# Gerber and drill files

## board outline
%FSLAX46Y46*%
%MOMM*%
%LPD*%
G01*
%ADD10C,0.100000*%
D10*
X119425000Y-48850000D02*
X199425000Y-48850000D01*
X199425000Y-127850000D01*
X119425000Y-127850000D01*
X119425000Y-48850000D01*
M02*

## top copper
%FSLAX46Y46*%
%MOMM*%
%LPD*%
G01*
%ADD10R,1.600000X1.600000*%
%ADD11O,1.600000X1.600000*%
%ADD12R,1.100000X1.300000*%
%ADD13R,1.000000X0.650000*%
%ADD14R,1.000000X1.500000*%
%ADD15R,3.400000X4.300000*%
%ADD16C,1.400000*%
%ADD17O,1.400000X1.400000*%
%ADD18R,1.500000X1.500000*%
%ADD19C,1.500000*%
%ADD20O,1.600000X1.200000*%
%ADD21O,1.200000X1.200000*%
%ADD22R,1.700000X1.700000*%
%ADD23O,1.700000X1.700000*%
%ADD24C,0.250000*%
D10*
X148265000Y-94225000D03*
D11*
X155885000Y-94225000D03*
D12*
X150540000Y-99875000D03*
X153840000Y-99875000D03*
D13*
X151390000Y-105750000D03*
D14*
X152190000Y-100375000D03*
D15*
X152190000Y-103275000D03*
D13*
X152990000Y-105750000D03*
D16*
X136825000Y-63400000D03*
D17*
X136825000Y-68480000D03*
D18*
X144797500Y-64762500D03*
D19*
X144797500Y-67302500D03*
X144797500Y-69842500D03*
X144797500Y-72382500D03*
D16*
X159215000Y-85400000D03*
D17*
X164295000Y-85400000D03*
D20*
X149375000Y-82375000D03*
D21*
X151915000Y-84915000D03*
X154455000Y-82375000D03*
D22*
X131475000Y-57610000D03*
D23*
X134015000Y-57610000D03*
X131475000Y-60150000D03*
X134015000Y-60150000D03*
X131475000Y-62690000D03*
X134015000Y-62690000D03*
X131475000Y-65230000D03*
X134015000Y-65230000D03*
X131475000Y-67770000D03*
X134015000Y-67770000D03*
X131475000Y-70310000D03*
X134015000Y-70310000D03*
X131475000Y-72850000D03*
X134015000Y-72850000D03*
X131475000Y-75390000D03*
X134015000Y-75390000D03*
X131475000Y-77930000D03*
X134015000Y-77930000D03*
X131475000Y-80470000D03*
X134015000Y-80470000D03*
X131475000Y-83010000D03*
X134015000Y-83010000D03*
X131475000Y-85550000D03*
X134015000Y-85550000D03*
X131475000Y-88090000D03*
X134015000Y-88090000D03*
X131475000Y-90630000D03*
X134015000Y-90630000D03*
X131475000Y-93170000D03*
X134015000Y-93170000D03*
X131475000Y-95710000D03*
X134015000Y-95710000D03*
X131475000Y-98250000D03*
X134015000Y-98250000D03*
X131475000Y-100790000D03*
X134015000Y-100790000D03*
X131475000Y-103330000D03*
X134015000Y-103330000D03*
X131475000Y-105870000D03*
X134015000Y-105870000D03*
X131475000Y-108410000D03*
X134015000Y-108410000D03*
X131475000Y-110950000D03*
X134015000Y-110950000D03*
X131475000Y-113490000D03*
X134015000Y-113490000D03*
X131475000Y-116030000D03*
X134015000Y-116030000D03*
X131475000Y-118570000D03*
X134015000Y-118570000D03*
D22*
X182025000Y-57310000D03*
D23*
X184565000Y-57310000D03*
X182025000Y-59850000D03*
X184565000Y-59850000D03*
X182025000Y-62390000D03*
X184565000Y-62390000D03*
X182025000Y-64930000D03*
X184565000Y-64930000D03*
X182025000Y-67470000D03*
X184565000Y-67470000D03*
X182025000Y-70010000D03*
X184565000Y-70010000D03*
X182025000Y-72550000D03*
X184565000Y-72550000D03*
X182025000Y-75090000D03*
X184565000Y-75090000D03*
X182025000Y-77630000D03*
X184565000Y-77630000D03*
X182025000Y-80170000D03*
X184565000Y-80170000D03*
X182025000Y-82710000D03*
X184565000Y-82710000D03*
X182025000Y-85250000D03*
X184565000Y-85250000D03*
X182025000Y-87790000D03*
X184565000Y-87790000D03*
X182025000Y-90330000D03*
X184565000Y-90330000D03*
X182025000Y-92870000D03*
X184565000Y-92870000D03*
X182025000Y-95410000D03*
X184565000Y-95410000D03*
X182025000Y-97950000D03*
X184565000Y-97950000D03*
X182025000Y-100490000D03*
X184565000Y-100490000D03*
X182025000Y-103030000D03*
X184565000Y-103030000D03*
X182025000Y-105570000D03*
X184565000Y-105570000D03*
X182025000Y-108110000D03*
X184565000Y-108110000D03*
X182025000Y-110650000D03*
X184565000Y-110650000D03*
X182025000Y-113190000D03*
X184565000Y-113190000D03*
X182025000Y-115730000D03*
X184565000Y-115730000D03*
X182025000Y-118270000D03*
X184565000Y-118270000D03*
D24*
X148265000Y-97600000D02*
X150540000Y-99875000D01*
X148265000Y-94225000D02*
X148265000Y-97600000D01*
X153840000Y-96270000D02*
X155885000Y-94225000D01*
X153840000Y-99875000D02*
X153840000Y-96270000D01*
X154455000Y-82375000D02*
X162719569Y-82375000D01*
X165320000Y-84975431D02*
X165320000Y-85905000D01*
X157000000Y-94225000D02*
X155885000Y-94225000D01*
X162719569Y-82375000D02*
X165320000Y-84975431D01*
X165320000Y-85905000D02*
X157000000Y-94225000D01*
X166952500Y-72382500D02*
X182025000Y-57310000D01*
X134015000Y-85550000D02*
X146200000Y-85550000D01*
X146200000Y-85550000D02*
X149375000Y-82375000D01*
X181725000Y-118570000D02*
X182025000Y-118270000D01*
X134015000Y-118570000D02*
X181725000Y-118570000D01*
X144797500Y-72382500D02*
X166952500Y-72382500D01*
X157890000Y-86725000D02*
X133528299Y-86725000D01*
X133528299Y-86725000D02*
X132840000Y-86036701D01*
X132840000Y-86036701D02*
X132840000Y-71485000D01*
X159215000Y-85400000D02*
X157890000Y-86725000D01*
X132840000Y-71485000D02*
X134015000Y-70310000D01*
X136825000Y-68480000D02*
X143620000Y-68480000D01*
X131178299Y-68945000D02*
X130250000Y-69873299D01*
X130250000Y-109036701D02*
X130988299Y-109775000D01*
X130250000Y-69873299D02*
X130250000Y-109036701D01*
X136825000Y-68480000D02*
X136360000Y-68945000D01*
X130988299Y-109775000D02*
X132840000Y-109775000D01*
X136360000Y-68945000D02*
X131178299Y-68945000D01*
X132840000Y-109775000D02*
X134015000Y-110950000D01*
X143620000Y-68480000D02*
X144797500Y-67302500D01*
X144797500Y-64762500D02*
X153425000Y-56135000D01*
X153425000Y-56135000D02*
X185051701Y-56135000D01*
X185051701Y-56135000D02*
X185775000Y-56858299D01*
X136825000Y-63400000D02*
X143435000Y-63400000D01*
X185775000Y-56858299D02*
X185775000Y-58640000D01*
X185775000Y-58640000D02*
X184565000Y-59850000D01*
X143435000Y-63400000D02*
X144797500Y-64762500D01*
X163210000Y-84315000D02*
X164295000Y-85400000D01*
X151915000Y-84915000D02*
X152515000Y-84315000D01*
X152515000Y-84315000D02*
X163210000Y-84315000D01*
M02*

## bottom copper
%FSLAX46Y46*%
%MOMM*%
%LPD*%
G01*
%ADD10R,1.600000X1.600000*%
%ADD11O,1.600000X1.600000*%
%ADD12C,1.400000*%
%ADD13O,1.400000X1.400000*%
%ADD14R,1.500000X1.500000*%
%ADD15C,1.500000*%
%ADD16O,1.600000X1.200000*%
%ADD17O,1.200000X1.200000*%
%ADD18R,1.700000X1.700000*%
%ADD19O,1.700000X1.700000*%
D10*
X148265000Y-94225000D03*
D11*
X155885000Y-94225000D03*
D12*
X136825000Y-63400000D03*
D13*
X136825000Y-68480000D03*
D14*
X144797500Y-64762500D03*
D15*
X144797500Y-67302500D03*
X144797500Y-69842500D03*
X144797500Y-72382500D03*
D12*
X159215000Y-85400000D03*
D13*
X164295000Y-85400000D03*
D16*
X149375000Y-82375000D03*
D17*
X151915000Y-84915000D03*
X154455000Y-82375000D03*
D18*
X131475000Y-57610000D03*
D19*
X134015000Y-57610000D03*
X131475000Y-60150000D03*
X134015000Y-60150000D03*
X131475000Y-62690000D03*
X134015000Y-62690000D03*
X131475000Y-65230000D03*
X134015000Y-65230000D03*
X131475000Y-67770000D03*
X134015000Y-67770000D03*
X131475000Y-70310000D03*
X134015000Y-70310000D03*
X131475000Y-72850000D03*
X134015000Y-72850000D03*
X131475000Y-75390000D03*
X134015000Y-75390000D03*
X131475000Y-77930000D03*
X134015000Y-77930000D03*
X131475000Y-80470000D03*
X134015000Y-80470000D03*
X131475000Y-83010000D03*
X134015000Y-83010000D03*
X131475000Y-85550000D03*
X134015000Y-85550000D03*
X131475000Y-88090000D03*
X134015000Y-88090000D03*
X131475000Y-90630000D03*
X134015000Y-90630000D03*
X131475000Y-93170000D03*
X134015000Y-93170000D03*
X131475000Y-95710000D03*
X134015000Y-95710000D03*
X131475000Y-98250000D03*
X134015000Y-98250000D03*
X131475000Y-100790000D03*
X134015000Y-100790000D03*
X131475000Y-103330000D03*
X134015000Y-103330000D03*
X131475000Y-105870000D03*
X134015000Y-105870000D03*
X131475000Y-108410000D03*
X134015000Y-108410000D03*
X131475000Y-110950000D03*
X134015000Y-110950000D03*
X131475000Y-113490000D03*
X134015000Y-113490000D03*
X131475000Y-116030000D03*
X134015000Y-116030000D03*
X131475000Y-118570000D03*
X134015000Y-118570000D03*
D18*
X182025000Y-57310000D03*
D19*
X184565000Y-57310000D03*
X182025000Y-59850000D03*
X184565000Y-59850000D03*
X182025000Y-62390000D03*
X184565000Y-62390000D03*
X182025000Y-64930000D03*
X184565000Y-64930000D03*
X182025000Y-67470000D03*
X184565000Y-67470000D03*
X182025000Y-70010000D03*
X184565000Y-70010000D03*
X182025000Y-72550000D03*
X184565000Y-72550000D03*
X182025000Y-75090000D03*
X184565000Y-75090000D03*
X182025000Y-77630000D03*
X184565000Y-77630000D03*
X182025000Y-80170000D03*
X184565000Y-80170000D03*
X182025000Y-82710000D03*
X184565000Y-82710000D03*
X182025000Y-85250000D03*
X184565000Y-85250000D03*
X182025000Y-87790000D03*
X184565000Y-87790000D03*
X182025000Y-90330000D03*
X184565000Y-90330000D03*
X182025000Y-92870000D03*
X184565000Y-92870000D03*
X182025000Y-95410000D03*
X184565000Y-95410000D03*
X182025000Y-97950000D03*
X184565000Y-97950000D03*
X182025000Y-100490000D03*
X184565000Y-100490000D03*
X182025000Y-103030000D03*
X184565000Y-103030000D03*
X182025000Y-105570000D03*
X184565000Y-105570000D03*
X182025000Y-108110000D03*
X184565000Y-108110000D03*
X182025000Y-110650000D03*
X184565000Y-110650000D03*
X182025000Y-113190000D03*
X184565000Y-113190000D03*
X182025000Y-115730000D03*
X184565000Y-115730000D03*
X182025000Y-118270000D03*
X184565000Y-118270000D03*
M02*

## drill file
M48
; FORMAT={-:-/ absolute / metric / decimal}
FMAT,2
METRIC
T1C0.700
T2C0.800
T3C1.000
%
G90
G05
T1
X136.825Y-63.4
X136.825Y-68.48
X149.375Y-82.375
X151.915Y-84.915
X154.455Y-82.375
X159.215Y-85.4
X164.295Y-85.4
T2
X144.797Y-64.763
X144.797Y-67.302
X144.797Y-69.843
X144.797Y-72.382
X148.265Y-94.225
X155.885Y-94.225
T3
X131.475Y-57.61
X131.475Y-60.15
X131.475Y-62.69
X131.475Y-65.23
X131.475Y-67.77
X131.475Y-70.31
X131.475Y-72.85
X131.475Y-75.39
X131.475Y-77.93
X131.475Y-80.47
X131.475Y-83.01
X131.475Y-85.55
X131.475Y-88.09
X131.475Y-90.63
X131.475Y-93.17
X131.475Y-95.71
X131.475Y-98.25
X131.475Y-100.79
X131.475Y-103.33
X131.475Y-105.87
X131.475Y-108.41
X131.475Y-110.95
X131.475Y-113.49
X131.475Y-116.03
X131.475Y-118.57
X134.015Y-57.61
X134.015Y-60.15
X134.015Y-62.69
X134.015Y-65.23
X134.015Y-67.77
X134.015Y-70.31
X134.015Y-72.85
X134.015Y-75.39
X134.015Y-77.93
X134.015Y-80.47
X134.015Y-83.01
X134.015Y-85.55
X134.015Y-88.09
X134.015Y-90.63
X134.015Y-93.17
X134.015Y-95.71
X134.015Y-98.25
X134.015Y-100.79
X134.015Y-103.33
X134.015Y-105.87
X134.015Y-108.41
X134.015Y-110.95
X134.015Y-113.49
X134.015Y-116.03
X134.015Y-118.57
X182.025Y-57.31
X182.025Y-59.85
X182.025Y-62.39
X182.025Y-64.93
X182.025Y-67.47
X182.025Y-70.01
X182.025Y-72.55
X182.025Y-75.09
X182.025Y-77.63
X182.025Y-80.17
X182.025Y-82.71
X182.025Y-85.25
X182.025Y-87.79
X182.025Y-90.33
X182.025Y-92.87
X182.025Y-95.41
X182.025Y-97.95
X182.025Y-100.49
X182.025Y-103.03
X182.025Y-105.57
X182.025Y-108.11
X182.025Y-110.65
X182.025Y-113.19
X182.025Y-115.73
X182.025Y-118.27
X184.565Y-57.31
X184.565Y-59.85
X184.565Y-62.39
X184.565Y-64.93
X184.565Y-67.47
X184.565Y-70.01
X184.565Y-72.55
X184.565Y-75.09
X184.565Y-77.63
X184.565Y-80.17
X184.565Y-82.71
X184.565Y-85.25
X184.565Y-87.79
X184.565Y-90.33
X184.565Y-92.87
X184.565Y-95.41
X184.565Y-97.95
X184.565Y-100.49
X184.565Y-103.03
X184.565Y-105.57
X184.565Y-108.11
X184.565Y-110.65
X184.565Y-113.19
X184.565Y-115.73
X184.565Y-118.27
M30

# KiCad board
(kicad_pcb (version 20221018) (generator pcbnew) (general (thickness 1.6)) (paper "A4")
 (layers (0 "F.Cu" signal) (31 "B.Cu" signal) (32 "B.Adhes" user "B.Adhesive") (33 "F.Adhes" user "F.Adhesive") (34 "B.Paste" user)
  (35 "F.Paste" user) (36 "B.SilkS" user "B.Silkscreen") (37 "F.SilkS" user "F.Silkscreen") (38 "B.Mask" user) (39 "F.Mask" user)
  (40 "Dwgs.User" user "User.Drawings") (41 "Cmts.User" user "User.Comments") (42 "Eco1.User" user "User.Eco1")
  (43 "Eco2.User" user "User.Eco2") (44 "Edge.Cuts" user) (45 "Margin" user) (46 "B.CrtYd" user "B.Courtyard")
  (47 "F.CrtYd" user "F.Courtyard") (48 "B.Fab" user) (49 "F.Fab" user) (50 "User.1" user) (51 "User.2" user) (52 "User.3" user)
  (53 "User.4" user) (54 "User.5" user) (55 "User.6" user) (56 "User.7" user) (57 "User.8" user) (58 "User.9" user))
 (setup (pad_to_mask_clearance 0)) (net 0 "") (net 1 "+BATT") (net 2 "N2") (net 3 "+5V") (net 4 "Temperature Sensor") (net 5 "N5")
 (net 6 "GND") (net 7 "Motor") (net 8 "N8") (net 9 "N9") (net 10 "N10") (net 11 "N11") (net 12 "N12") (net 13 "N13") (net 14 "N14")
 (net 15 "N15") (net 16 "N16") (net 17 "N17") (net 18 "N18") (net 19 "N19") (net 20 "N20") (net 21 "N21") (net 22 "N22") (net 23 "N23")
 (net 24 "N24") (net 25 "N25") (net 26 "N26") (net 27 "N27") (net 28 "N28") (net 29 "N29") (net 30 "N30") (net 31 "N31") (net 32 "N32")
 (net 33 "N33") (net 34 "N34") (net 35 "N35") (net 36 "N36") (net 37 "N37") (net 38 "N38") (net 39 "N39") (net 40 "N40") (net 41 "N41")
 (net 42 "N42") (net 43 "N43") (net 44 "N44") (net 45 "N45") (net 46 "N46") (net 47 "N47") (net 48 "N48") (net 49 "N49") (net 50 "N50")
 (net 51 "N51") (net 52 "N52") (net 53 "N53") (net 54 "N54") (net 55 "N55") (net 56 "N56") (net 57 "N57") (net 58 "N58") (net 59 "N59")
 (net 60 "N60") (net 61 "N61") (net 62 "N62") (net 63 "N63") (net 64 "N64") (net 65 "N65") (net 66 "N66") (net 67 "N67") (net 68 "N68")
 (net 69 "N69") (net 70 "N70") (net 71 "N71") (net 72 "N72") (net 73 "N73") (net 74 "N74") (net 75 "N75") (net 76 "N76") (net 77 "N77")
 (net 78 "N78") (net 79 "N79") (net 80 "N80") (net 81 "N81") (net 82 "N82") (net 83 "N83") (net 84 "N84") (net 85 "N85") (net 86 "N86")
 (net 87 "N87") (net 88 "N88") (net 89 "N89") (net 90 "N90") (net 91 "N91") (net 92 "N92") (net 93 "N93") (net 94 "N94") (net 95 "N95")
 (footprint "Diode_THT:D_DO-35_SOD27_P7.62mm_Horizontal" (layer "F.Cu") (at 148.265 94.225)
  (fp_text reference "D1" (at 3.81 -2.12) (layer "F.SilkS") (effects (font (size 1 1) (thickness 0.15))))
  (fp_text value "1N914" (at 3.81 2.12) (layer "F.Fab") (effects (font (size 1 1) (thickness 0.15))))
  (pad "1" thru_hole rect (at 0 0) (size 1.6 1.6) (drill 0.8) (layers "*.Cu" "*.Mask") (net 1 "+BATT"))
  (pad "2" thru_hole oval (at 7.62 0) (size 1.6 1.6) (drill 0.8) (layers "*.Cu" "*.Mask") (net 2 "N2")))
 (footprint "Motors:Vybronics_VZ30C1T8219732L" (layer "F.Cu") (at 152.19 104.225)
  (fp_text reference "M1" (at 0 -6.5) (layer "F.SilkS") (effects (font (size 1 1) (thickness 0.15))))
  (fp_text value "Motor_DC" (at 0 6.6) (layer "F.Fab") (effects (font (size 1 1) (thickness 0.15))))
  (pad "" smd rect (at -0.85 -2.315 270) (size 1.07 1.4) (layers "F.Paste"))
  (pad "" smd rect (at -0.85 -0.905 270) (size 1.07 1.4) (layers "F.Paste"))
  (pad "" smd rect (at -0.85 0.505 270) (size 1.07 1.4) (layers "F.Paste"))
  (pad "" smd rect (at 0.85 -2.315 270) (size 1.07 1.4) (layers "F.Paste"))
  (pad "" smd rect (at 0.85 -0.905 270) (size 1.07 1.4) (layers "F.Paste"))
  (pad "" smd rect (at 0.85 0.505 270) (size 1.07 1.4) (layers "F.Paste"))
  (pad "1" smd rect (at -1.65 -4.35 270) (size 1.3 1.1) (layers "F.Cu" "F.Paste" "F.Mask") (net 1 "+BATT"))
  (pad "2" smd rect (at 1.65 -4.35 270) (size 1.3 1.1) (layers "F.Cu" "F.Paste" "F.Mask") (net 2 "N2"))
  (pad "SH" smd rect (at -0.8 1.525) (size 1 0.65) (layers "F.Cu" "F.Paste" "F.Mask"))
  (pad "SH" smd rect (at 0 -3.85 270) (size 1.5 1) (layers "F.Cu" "F.Paste" "F.Mask"))
  (pad "SH" smd rect (at 0 -0.95 270) (size 4.3 3.4) (layers "F.Cu" "F.Mask"))
  (pad "SH" smd rect (at 0.8 1.525) (size 1 0.65) (layers "F.Cu" "F.Paste" "F.Mask")))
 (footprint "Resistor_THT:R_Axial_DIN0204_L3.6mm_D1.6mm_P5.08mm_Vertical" (layer "F.Cu") (at 136.825 63.4 -90)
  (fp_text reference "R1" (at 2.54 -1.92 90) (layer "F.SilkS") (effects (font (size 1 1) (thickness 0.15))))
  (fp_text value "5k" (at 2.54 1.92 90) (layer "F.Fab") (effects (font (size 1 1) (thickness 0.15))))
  (pad "1" thru_hole circle (at 0 0 270) (size 1.4 1.4) (drill 0.7) (layers "*.Cu" "*.Mask") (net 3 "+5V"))
  (pad "2" thru_hole oval (at 5.08 0 270) (size 1.4 1.4) (drill 0.7) (layers "*.Cu" "*.Mask") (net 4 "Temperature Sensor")))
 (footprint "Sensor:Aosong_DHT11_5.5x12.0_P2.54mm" (layer "F.Cu") (at 144.7975 64.7625)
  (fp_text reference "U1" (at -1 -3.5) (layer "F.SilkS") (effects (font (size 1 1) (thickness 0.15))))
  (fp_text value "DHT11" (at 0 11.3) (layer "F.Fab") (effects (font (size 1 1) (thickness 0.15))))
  (pad "1" thru_hole rect (at 0 0) (size 1.5 1.5) (drill 0.8) (layers "*.Cu" "*.Mask") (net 3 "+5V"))
  (pad "2" thru_hole circle (at 0 2.54) (size 1.5 1.5) (drill 0.8) (layers "*.Cu" "*.Mask") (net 4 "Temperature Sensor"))
  (pad "3" thru_hole circle (at 0 5.08) (size 1.5 1.5) (drill 0.8) (layers "*.Cu" "*.Mask") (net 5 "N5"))
  (pad "4" thru_hole circle (at 0 7.62) (size 1.5 1.5) (drill 0.8) (layers "*.Cu" "*.Mask") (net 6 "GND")))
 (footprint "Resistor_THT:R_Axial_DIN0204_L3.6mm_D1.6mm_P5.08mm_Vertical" (layer "F.Cu") (at 159.215 85.4)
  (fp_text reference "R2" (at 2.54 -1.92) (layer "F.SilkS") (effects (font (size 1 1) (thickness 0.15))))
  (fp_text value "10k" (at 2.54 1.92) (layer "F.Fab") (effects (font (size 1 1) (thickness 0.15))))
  (pad "1" thru_hole circle (at 0 0) (size 1.4 1.4) (drill 0.7) (layers "*.Cu" "*.Mask") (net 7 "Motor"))
  (pad "2" thru_hole oval (at 5.08 0) (size 1.4 1.4) (drill 0.7) (layers "*.Cu" "*.Mask") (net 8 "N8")))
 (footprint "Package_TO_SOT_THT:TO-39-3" (layer "F.Cu") (at 149.375 82.375)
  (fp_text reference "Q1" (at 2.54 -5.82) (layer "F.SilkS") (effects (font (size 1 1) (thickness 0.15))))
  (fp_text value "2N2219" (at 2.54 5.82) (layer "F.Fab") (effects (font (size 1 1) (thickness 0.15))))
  (pad "1" thru_hole oval (at 0 0) (size 1.6 1.2) (drill 0.7) (layers "*.Cu" "*.Mask") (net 6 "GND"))
  (pad "2" thru_hole oval (at 2.54 2.54) (size 1.2 1.2) (drill 0.7) (layers "*.Cu" "*.Mask") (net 8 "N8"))
  (pad "3" thru_hole oval (at 5.08 0) (size 1.2 1.2) (drill 0.7) (layers "*.Cu" "*.Mask") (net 2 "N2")))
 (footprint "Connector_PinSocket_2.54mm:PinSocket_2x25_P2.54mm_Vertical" (layer "B.Cu") (at 131.475 57.61 180)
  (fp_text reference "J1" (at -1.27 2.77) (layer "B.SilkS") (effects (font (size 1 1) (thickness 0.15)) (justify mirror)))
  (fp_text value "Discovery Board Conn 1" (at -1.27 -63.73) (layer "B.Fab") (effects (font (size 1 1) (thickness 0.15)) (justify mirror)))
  (pad "1" thru_hole rect (at 0 0 180) (size 1.7 1.7) (drill 1) (layers "*.Cu" "*.Mask") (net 6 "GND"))
  (pad "2" thru_hole oval (at -2.54 0 180) (size 1.7 1.7) (drill 1) (layers "*.Cu" "*.Mask") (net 6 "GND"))
  (pad "3" thru_hole oval (at 0 -2.54 180) (size 1.7 1.7) (drill 1) (layers "*.Cu" "*.Mask") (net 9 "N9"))
  (pad "4" thru_hole oval (at -2.54 -2.54 180) (size 1.7 1.7) (drill 1) (layers "*.Cu" "*.Mask") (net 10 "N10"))
  (pad "5" thru_hole oval (at 0 -5.08 180) (size 1.7 1.7) (drill 1) (layers "*.Cu" "*.Mask") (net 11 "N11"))
  (pad "6" thru_hole oval (at -2.54 -5.08 180) (size 1.7 1.7) (drill 1) (layers "*.Cu" "*.Mask") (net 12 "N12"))
  (pad "7" thru_hole oval (at 0 -7.62 180) (size 1.7 1.7) (drill 1) (layers "*.Cu" "*.Mask") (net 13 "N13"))
  (pad "8" thru_hole oval (at -2.54 -7.62 180) (size 1.7 1.7) (drill 1) (layers "*.Cu" "*.Mask") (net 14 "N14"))
  (pad "9" thru_hole oval (at 0 -10.16 180) (size 1.7 1.7) (drill 1) (layers "*.Cu" "*.Mask") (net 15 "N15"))
  (pad "10" thru_hole oval (at -2.54 -10.16 180) (size 1.7 1.7) (drill 1) (layers "*.Cu" "*.Mask") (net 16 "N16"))
  (pad "11" thru_hole oval (at 0 -12.7 180) (size 1.7 1.7) (drill 1) (layers "*.Cu" "*.Mask") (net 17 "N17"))
  (pad "12" thru_hole oval (at -2.54 -12.7 180) (size 1.7 1.7) (drill 1) (layers "*.Cu" "*.Mask") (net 7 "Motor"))
  (pad "13" thru_hole oval (at 0 -15.24 180) (size 1.7 1.7) (drill 1) (layers "*.Cu" "*.Mask") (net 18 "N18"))
  (pad "14" thru_hole oval (at -2.54 -15.24 180) (size 1.7 1.7) (drill 1) (layers "*.Cu" "*.Mask") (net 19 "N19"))
  (pad "15" thru_hole oval (at 0 -17.78 180) (size 1.7 1.7) (drill 1) (layers "*.Cu" "*.Mask") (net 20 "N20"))
  (pad "16" thru_hole oval (at -2.54 -17.78 180) (size 1.7 1.7) (drill 1) (layers "*.Cu" "*.Mask") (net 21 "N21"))
  (pad "17" thru_hole oval (at 0 -20.32 180) (size 1.7 1.7) (drill 1) (layers "*.Cu" "*.Mask") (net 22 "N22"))
  (pad "18" thru_hole oval (at -2.54 -20.32 180) (size 1.7 1.7) (drill 1) (layers "*.Cu" "*.Mask") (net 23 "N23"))
  (pad "19" thru_hole oval (at 0 -22.86 180) (size 1.7 1.7) (drill 1) (layers "*.Cu" "*.Mask") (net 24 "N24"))
  (pad "20" thru_hole oval (at -2.54 -22.86 180) (size 1.7 1.7) (drill 1) (layers "*.Cu" "*.Mask") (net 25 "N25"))
  (pad "21" thru_hole oval (at 0 -25.4 180) (size 1.7 1.7) (drill 1) (layers "*.Cu" "*.Mask") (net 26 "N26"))
  (pad "22" thru_hole oval (at -2.54 -25.4 180) (size 1.7 1.7) (drill 1) (layers "*.Cu" "*.Mask") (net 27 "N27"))
  (pad "23" thru_hole oval (at 0 -27.94 180) (size 1.7 1.7) (drill 1) (layers "*.Cu" "*.Mask") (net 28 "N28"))
  (pad "24" thru_hole oval (at -2.54 -27.94 180) (size 1.7 1.7) (drill 1) (layers "*.Cu" "*.Mask") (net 6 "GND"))
  (pad "25" thru_hole oval (at 0 -30.48 180) (size 1.7 1.7) (drill 1) (layers "*.Cu" "*.Mask") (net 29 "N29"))
  (pad "26" thru_hole oval (at -2.54 -30.48 180) (size 1.7 1.7) (drill 1) (layers "*.Cu" "*.Mask") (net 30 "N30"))
  (pad "27" thru_hole oval (at 0 -33.02 180) (size 1.7 1.7) (drill 1) (layers "*.Cu" "*.Mask") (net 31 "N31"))
  (pad "28" thru_hole oval (at -2.54 -33.02 180) (size 1.7 1.7) (drill 1) (layers "*.Cu" "*.Mask") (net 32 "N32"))
  (pad "29" thru_hole oval (at 0 -35.56 180) (size 1.7 1.7) (drill 1) (layers "*.Cu" "*.Mask") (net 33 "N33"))
  (pad "30" thru_hole oval (at -2.54 -35.56 180) (size 1.7 1.7) (drill 1) (layers "*.Cu" "*.Mask") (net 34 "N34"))
  (pad "31" thru_hole oval (at 0 -38.1 180) (size 1.7 1.7) (drill 1) (layers "*.Cu" "*.Mask") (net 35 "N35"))
  (pad "32" thru_hole oval (at -2.54 -38.1 180) (size 1.7 1.7) (drill 1) (layers "*.Cu" "*.Mask") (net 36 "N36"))
  (pad "33" thru_hole oval (at 0 -40.64 180) (size 1.7 1.7) (drill 1) (layers "*.Cu" "*.Mask") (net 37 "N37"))
  (pad "34" thru_hole oval (at -2.54 -40.64 180) (size 1.7 1.7) (drill 1) (layers "*.Cu" "*.Mask") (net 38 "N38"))
  (pad "35" thru_hole oval (at 0 -43.18 180) (size 1.7 1.7) (drill 1) (layers "*.Cu" "*.Mask") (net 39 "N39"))
  (pad "36" thru_hole oval (at -2.54 -43.18 180) (size 1.7 1.7) (drill 1) (layers "*.Cu" "*.Mask") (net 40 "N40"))
  (pad "37" thru_hole oval (at 0 -45.72 180) (size 1.7 1.7) (drill 1) (layers "*.Cu" "*.Mask") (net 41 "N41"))
  (pad "38" thru_hole oval (at -2.54 -45.72 180) (size 1.7 1.7) (drill 1) (layers "*.Cu" "*.Mask") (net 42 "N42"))
  (pad "39" thru_hole oval (at 0 -48.26 180) (size 1.7 1.7) (drill 1) (layers "*.Cu" "*.Mask") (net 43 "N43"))
  (pad "40" thru_hole oval (at -2.54 -48.26 180) (size 1.7 1.7) (drill 1) (layers "*.Cu" "*.Mask") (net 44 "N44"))
  (pad "41" thru_hole oval (at 0 -50.8 180) (size 1.7 1.7) (drill 1) (layers "*.Cu" "*.Mask") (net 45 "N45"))
  (pad "42" thru_hole oval (at -2.54 -50.8 180) (size 1.7 1.7) (drill 1) (layers "*.Cu" "*.Mask") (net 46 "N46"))
  (pad "43" thru_hole oval (at 0 -53.34 180) (size 1.7 1.7) (drill 1) (layers "*.Cu" "*.Mask") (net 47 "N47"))
  (pad "44" thru_hole oval (at -2.54 -53.34 180) (size 1.7 1.7) (drill 1) (layers "*.Cu" "*.Mask") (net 4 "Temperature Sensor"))
  (pad "45" thru_hole oval (at 0 -55.88 180) (size 1.7 1.7) (drill 1) (layers "*.Cu" "*.Mask") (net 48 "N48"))
  (pad "46" thru_hole oval (at -2.54 -55.88 180) (size 1.7 1.7) (drill 1) (layers "*.Cu" "*.Mask") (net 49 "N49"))
  (pad "47" thru_hole oval (at 0 -58.42 180) (size 1.7 1.7) (drill 1) (layers "*.Cu" "*.Mask") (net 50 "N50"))
  (pad "48" thru_hole oval (at -2.54 -58.42 180) (size 1.7 1.7) (drill 1) (layers "*.Cu" "*.Mask") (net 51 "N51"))
  (pad "49" thru_hole oval (at 0 -60.96 180) (size 1.7 1.7) (drill 1) (layers "*.Cu" "*.Mask") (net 6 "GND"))
  (pad "50" thru_hole oval (at -2.54 -60.96 180) (size 1.7 1.7) (drill 1) (layers "*.Cu" "*.Mask") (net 6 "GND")))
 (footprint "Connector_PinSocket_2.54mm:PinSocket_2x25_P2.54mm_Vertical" (layer "B.Cu") (at 182.025 57.31 180)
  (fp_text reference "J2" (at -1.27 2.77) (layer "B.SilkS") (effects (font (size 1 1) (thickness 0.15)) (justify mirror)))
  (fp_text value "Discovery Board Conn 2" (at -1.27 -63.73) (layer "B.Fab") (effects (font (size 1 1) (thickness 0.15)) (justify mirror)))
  (pad "1" thru_hole rect (at 0 0 180) (size 1.7 1.7) (drill 1) (layers "*.Cu" "*.Mask") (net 6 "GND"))
  (pad "2" thru_hole oval (at -2.54 0 180) (size 1.7 1.7) (drill 1) (layers "*.Cu" "*.Mask") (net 6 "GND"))
  (pad "3" thru_hole oval (at 0 -2.54 180) (size 1.7 1.7) (drill 1) (layers "*.Cu" "*.Mask") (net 3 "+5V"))
  (pad "4" thru_hole oval (at -2.54 -2.54 180) (size 1.7 1.7) (drill 1) (layers "*.Cu" "*.Mask") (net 3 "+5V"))
  (pad "5" thru_hole oval (at 0 -5.08 180) (size 1.7 1.7) (drill 1) (layers "*.Cu" "*.Mask") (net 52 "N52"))
  (pad "6" thru_hole oval (at -2.54 -5.08 180) (size 1.7 1.7) (drill 1) (layers "*.Cu" "*.Mask") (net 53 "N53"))
  (pad "7" thru_hole oval (at 0 -7.62 180) (size 1.7 1.7) (drill 1) (layers "*.Cu" "*.Mask") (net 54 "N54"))
  (pad "8" thru_hole oval (at -2.54 -7.62 180) (size 1.7 1.7) (drill 1) (layers "*.Cu" "*.Mask") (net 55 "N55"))
  (pad "9" thru_hole oval (at 0 -10.16 180) (size 1.7 1.7) (drill 1) (layers "*.Cu" "*.Mask") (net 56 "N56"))
  (pad "10" thru_hole oval (at -2.54 -10.16 180) (size 1.7 1.7) (drill 1) (layers "*.Cu" "*.Mask") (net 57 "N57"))
  (pad "11" thru_hole oval (at 0 -12.7 180) (size 1.7 1.7) (drill 1) (layers "*.Cu" "*.Mask") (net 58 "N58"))
  (pad "12" thru_hole oval (at -2.54 -12.7 180) (size 1.7 1.7) (drill 1) (layers "*.Cu" "*.Mask") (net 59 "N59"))
  (pad "13" thru_hole oval (at 0 -15.24 180) (size 1.7 1.7) (drill 1) (layers "*.Cu" "*.Mask") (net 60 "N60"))
  (pad "14" thru_hole oval (at -2.54 -15.24 180) (size 1.7 1.7) (drill 1) (layers "*.Cu" "*.Mask") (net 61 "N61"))
  (pad "15" thru_hole oval (at 0 -17.78 180) (size 1.7 1.7) (drill 1) (layers "*.Cu" "*.Mask") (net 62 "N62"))
  (pad "16" thru_hole oval (at -2.54 -17.78 180) (size 1.7 1.7) (drill 1) (layers "*.Cu" "*.Mask") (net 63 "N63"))
  (pad "17" thru_hole oval (at 0 -20.32 180) (size 1.7 1.7) (drill 1) (layers "*.Cu" "*.Mask") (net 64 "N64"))
  (pad "18" thru_hole oval (at -2.54 -20.32 180) (size 1.7 1.7) (drill 1) (layers "*.Cu" "*.Mask") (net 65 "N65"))
  (pad "19" thru_hole oval (at 0 -22.86 180) (size 1.7 1.7) (drill 1) (layers "*.Cu" "*.Mask") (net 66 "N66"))
  (pad "20" thru_hole oval (at -2.54 -22.86 180) (size 1.7 1.7) (drill 1) (layers "*.Cu" "*.Mask") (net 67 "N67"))
  (pad "21" thru_hole oval (at 0 -25.4 180) (size 1.7 1.7) (drill 1) (layers "*.Cu" "*.Mask") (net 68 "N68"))
  (pad "22" thru_hole oval (at -2.54 -25.4 180) (size 1.7 1.7) (drill 1) (layers "*.Cu" "*.Mask") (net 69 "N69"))
  (pad "23" thru_hole oval (at 0 -27.94 180) (size 1.7 1.7) (drill 1) (layers "*.Cu" "*.Mask") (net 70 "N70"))
  (pad "24" thru_hole oval (at -2.54 -27.94 180) (size 1.7 1.7) (drill 1) (layers "*.Cu" "*.Mask") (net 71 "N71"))
  (pad "25" thru_hole oval (at 0 -30.48 180) (size 1.7 1.7) (drill 1) (layers "*.Cu" "*.Mask") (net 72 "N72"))
  (pad "26" thru_hole oval (at -2.54 -30.48 180) (size 1.7 1.7) (drill 1) (layers "*.Cu" "*.Mask") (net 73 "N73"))
  (pad "27" thru_hole oval (at 0 -33.02 180) (size 1.7 1.7) (drill 1) (layers "*.Cu" "*.Mask") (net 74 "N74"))
  (pad "28" thru_hole oval (at -2.54 -33.02 180) (size 1.7 1.7) (drill 1) (layers "*.Cu" "*.Mask") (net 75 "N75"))
  (pad "29" thru_hole oval (at 0 -35.56 180) (size 1.7 1.7) (drill 1) (layers "*.Cu" "*.Mask") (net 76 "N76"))
  (pad "30" thru_hole oval (at -2.54 -35.56 180) (size 1.7 1.7) (drill 1) (layers "*.Cu" "*.Mask") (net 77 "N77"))
  (pad "31" thru_hole oval (at 0 -38.1 180) (size 1.7 1.7) (drill 1) (layers "*.Cu" "*.Mask") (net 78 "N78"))
  (pad "32" thru_hole oval (at -2.54 -38.1 180) (size 1.7 1.7) (drill 1) (layers "*.Cu" "*.Mask") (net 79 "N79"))
  (pad "33" thru_hole oval (at 0 -40.64 180) (size 1.7 1.7) (drill 1) (layers "*.Cu" "*.Mask") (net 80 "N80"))
  (pad "34" thru_hole oval (at -2.54 -40.64 180) (size 1.7 1.7) (drill 1) (layers "*.Cu" "*.Mask") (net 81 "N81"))
  (pad "35" thru_hole oval (at 0 -43.18 180) (size 1.7 1.7) (drill 1) (layers "*.Cu" "*.Mask") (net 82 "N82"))
  (pad "36" thru_hole oval (at -2.54 -43.18 180) (size 1.7 1.7) (drill 1) (layers "*.Cu" "*.Mask") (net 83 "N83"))
  (pad "37" thru_hole oval (at 0 -45.72 180) (size 1.7 1.7) (drill 1) (layers "*.Cu" "*.Mask") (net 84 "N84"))
  (pad "38" thru_hole oval (at -2.54 -45.72 180) (size 1.7 1.7) (drill 1) (layers "*.Cu" "*.Mask") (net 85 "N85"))
  (pad "39" thru_hole oval (at 0 -48.26 180) (size 1.7 1.7) (drill 1) (layers "*.Cu" "*.Mask") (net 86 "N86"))
  (pad "40" thru_hole oval (at -2.54 -48.26 180) (size 1.7 1.7) (drill 1) (layers "*.Cu" "*.Mask") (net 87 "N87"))
  (pad "41" thru_hole oval (at 0 -50.8 180) (size 1.7 1.7) (drill 1) (layers "*.Cu" "*.Mask") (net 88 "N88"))
  (pad "42" thru_hole oval (at -2.54 -50.8 180) (size 1.7 1.7) (drill 1) (layers "*.Cu" "*.Mask") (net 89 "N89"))
  (pad "43" thru_hole oval (at 0 -53.34 180) (size 1.7 1.7) (drill 1) (layers "*.Cu" "*.Mask") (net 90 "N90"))
  (pad "44" thru_hole oval (at -2.54 -53.34 180) (size 1.7 1.7) (drill 1) (layers "*.Cu" "*.Mask") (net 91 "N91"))
  (pad "45" thru_hole oval (at 0 -55.88 180) (size 1.7 1.7) (drill 1) (layers "*.Cu" "*.Mask") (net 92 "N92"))
  (pad "46" thru_hole oval (at -2.54 -55.88 180) (size 1.7 1.7) (drill 1) (layers "*.Cu" "*.Mask") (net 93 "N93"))
  (pad "47" thru_hole oval (at 0 -58.42 180) (size 1.7 1.7) (drill 1) (layers "*.Cu" "*.Mask") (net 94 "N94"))
  (pad "48" thru_hole oval (at -2.54 -58.42 180) (size 1.7 1.7) (drill 1) (layers "*.Cu" "*.Mask") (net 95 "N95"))
  (pad "49" thru_hole oval (at 0 -60.96 180) (size 1.7 1.7) (drill 1) (layers "*.Cu" "*.Mask") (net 6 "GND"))
  (pad "50" thru_hole oval (at -2.54 -60.96 180) (size 1.7 1.7) (drill 1) (layers "*.Cu" "*.Mask") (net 6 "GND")))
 (gr_rect (start 119.425 48.85) (end 199.425 127.85) (stroke (width 0.1) (type default)) (fill none) (layer "Edge.Cuts"))
 (segment (start 148.265 97.6) (end 150.54 99.875) (width 0.25) (layer "F.Cu") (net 1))
 (segment (start 148.265 94.225) (end 148.265 97.6) (width 0.25) (layer "F.Cu") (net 1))
 (segment (start 153.84 96.27) (end 155.885 94.225) (width 0.25) (layer "F.Cu") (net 2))
 (segment (start 153.84 99.875) (end 153.84 96.27) (width 0.25) (layer "F.Cu") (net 2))
 (segment (start 154.455 82.375) (end 162.719569 82.375) (width 0.25) (layer "F.Cu") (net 2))
 (segment (start 165.32 84.975431) (end 165.32 85.905) (width 0.25) (layer "F.Cu") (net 2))
 (segment (start 157 94.225) (end 155.885 94.225) (width 0.25) (layer "F.Cu") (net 2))
 (segment (start 162.719569 82.375) (end 165.32 84.975431) (width 0.25) (layer "F.Cu") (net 2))
 (segment (start 165.32 85.905) (end 157 94.225) (width 0.25) (layer "F.Cu") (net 2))
 (segment (start 166.9525 72.3825) (end 182.025 57.31) (width 0.25) (layer "F.Cu") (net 6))
 (segment (start 134.015 85.55) (end 146.2 85.55) (width 0.25) (layer "F.Cu") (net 6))
 (segment (start 146.2 85.55) (end 149.375 82.375) (width 0.25) (layer "F.Cu") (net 6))
 (segment (start 181.725 118.57) (end 182.025 118.27) (width 0.25) (layer "F.Cu") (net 6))
 (segment (start 134.015 118.57) (end 181.725 118.57) (width 0.25) (layer "F.Cu") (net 6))
 (segment (start 144.7975 72.3825) (end 166.9525 72.3825) (width 0.25) (layer "F.Cu") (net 6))
 (segment (start 157.89 86.725) (end 133.528299 86.725) (width 0.25) (layer "F.Cu") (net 7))
 (segment (start 133.528299 86.725) (end 132.84 86.036701) (width 0.25) (layer "F.Cu") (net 7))
 (segment (start 132.84 86.036701) (end 132.84 71.485) (width 0.25) (layer "F.Cu") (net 7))
 (segment (start 159.215 85.4) (end 157.89 86.725) (width 0.25) (layer "F.Cu") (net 7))
 (segment (start 132.84 71.485) (end 134.015 70.31) (width 0.25) (layer "F.Cu") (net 7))
 (segment (start 136.825 68.48) (end 143.62 68.48) (width 0.25) (layer "F.Cu") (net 4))
 (segment (start 131.178299 68.945) (end 130.25 69.873299) (width 0.25) (layer "F.Cu") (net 4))
 (segment (start 130.25 109.036701) (end 130.988299 109.775) (width 0.25) (layer "F.Cu") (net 4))
 (segment (start 130.25 69.873299) (end 130.25 109.036701) (width 0.25) (layer "F.Cu") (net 4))
 (segment (start 136.825 68.48) (end 136.36 68.945) (width 0.25) (layer "F.Cu") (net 4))
 (segment (start 130.988299 109.775) (end 132.84 109.775) (width 0.25) (layer "F.Cu") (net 4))
 (segment (start 136.36 68.945) (end 131.178299 68.945) (width 0.25) (layer "F.Cu") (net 4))
 (segment (start 132.84 109.775) (end 134.015 110.95) (width 0.25) (layer "F.Cu") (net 4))
 (segment (start 143.62 68.48) (end 144.7975 67.3025) (width 0.25) (layer "F.Cu") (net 4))
 (segment (start 144.7975 64.7625) (end 153.425 56.135) (width 0.25) (layer "F.Cu") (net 3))
 (segment (start 153.425 56.135) (end 185.051701 56.135) (width 0.25) (layer "F.Cu") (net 3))
 (segment (start 185.051701 56.135) (end 185.775 56.858299) (width 0.25) (layer "F.Cu") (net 3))
 (segment (start 136.825 63.4) (end 143.435 63.4) (width 0.25) (layer "F.Cu") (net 3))
 (segment (start 185.775 56.858299) (end 185.775 58.64) (width 0.25) (layer "F.Cu") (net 3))
 (segment (start 185.775 58.64) (end 184.565 59.85) (width 0.25) (layer "F.Cu") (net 3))
 (segment (start 143.435 63.4) (end 144.7975 64.7625) (width 0.25) (layer "F.Cu") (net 3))
 (segment (start 163.21 84.315) (end 164.295 85.4) (width 0.25) (layer "F.Cu") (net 8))
 (segment (start 151.915 84.915) (end 152.515 84.315) (width 0.25) (layer "F.Cu") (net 8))
 (segment (start 152.515 84.315) (end 163.21 84.315) (width 0.25) (layer "F.Cu") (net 8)))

